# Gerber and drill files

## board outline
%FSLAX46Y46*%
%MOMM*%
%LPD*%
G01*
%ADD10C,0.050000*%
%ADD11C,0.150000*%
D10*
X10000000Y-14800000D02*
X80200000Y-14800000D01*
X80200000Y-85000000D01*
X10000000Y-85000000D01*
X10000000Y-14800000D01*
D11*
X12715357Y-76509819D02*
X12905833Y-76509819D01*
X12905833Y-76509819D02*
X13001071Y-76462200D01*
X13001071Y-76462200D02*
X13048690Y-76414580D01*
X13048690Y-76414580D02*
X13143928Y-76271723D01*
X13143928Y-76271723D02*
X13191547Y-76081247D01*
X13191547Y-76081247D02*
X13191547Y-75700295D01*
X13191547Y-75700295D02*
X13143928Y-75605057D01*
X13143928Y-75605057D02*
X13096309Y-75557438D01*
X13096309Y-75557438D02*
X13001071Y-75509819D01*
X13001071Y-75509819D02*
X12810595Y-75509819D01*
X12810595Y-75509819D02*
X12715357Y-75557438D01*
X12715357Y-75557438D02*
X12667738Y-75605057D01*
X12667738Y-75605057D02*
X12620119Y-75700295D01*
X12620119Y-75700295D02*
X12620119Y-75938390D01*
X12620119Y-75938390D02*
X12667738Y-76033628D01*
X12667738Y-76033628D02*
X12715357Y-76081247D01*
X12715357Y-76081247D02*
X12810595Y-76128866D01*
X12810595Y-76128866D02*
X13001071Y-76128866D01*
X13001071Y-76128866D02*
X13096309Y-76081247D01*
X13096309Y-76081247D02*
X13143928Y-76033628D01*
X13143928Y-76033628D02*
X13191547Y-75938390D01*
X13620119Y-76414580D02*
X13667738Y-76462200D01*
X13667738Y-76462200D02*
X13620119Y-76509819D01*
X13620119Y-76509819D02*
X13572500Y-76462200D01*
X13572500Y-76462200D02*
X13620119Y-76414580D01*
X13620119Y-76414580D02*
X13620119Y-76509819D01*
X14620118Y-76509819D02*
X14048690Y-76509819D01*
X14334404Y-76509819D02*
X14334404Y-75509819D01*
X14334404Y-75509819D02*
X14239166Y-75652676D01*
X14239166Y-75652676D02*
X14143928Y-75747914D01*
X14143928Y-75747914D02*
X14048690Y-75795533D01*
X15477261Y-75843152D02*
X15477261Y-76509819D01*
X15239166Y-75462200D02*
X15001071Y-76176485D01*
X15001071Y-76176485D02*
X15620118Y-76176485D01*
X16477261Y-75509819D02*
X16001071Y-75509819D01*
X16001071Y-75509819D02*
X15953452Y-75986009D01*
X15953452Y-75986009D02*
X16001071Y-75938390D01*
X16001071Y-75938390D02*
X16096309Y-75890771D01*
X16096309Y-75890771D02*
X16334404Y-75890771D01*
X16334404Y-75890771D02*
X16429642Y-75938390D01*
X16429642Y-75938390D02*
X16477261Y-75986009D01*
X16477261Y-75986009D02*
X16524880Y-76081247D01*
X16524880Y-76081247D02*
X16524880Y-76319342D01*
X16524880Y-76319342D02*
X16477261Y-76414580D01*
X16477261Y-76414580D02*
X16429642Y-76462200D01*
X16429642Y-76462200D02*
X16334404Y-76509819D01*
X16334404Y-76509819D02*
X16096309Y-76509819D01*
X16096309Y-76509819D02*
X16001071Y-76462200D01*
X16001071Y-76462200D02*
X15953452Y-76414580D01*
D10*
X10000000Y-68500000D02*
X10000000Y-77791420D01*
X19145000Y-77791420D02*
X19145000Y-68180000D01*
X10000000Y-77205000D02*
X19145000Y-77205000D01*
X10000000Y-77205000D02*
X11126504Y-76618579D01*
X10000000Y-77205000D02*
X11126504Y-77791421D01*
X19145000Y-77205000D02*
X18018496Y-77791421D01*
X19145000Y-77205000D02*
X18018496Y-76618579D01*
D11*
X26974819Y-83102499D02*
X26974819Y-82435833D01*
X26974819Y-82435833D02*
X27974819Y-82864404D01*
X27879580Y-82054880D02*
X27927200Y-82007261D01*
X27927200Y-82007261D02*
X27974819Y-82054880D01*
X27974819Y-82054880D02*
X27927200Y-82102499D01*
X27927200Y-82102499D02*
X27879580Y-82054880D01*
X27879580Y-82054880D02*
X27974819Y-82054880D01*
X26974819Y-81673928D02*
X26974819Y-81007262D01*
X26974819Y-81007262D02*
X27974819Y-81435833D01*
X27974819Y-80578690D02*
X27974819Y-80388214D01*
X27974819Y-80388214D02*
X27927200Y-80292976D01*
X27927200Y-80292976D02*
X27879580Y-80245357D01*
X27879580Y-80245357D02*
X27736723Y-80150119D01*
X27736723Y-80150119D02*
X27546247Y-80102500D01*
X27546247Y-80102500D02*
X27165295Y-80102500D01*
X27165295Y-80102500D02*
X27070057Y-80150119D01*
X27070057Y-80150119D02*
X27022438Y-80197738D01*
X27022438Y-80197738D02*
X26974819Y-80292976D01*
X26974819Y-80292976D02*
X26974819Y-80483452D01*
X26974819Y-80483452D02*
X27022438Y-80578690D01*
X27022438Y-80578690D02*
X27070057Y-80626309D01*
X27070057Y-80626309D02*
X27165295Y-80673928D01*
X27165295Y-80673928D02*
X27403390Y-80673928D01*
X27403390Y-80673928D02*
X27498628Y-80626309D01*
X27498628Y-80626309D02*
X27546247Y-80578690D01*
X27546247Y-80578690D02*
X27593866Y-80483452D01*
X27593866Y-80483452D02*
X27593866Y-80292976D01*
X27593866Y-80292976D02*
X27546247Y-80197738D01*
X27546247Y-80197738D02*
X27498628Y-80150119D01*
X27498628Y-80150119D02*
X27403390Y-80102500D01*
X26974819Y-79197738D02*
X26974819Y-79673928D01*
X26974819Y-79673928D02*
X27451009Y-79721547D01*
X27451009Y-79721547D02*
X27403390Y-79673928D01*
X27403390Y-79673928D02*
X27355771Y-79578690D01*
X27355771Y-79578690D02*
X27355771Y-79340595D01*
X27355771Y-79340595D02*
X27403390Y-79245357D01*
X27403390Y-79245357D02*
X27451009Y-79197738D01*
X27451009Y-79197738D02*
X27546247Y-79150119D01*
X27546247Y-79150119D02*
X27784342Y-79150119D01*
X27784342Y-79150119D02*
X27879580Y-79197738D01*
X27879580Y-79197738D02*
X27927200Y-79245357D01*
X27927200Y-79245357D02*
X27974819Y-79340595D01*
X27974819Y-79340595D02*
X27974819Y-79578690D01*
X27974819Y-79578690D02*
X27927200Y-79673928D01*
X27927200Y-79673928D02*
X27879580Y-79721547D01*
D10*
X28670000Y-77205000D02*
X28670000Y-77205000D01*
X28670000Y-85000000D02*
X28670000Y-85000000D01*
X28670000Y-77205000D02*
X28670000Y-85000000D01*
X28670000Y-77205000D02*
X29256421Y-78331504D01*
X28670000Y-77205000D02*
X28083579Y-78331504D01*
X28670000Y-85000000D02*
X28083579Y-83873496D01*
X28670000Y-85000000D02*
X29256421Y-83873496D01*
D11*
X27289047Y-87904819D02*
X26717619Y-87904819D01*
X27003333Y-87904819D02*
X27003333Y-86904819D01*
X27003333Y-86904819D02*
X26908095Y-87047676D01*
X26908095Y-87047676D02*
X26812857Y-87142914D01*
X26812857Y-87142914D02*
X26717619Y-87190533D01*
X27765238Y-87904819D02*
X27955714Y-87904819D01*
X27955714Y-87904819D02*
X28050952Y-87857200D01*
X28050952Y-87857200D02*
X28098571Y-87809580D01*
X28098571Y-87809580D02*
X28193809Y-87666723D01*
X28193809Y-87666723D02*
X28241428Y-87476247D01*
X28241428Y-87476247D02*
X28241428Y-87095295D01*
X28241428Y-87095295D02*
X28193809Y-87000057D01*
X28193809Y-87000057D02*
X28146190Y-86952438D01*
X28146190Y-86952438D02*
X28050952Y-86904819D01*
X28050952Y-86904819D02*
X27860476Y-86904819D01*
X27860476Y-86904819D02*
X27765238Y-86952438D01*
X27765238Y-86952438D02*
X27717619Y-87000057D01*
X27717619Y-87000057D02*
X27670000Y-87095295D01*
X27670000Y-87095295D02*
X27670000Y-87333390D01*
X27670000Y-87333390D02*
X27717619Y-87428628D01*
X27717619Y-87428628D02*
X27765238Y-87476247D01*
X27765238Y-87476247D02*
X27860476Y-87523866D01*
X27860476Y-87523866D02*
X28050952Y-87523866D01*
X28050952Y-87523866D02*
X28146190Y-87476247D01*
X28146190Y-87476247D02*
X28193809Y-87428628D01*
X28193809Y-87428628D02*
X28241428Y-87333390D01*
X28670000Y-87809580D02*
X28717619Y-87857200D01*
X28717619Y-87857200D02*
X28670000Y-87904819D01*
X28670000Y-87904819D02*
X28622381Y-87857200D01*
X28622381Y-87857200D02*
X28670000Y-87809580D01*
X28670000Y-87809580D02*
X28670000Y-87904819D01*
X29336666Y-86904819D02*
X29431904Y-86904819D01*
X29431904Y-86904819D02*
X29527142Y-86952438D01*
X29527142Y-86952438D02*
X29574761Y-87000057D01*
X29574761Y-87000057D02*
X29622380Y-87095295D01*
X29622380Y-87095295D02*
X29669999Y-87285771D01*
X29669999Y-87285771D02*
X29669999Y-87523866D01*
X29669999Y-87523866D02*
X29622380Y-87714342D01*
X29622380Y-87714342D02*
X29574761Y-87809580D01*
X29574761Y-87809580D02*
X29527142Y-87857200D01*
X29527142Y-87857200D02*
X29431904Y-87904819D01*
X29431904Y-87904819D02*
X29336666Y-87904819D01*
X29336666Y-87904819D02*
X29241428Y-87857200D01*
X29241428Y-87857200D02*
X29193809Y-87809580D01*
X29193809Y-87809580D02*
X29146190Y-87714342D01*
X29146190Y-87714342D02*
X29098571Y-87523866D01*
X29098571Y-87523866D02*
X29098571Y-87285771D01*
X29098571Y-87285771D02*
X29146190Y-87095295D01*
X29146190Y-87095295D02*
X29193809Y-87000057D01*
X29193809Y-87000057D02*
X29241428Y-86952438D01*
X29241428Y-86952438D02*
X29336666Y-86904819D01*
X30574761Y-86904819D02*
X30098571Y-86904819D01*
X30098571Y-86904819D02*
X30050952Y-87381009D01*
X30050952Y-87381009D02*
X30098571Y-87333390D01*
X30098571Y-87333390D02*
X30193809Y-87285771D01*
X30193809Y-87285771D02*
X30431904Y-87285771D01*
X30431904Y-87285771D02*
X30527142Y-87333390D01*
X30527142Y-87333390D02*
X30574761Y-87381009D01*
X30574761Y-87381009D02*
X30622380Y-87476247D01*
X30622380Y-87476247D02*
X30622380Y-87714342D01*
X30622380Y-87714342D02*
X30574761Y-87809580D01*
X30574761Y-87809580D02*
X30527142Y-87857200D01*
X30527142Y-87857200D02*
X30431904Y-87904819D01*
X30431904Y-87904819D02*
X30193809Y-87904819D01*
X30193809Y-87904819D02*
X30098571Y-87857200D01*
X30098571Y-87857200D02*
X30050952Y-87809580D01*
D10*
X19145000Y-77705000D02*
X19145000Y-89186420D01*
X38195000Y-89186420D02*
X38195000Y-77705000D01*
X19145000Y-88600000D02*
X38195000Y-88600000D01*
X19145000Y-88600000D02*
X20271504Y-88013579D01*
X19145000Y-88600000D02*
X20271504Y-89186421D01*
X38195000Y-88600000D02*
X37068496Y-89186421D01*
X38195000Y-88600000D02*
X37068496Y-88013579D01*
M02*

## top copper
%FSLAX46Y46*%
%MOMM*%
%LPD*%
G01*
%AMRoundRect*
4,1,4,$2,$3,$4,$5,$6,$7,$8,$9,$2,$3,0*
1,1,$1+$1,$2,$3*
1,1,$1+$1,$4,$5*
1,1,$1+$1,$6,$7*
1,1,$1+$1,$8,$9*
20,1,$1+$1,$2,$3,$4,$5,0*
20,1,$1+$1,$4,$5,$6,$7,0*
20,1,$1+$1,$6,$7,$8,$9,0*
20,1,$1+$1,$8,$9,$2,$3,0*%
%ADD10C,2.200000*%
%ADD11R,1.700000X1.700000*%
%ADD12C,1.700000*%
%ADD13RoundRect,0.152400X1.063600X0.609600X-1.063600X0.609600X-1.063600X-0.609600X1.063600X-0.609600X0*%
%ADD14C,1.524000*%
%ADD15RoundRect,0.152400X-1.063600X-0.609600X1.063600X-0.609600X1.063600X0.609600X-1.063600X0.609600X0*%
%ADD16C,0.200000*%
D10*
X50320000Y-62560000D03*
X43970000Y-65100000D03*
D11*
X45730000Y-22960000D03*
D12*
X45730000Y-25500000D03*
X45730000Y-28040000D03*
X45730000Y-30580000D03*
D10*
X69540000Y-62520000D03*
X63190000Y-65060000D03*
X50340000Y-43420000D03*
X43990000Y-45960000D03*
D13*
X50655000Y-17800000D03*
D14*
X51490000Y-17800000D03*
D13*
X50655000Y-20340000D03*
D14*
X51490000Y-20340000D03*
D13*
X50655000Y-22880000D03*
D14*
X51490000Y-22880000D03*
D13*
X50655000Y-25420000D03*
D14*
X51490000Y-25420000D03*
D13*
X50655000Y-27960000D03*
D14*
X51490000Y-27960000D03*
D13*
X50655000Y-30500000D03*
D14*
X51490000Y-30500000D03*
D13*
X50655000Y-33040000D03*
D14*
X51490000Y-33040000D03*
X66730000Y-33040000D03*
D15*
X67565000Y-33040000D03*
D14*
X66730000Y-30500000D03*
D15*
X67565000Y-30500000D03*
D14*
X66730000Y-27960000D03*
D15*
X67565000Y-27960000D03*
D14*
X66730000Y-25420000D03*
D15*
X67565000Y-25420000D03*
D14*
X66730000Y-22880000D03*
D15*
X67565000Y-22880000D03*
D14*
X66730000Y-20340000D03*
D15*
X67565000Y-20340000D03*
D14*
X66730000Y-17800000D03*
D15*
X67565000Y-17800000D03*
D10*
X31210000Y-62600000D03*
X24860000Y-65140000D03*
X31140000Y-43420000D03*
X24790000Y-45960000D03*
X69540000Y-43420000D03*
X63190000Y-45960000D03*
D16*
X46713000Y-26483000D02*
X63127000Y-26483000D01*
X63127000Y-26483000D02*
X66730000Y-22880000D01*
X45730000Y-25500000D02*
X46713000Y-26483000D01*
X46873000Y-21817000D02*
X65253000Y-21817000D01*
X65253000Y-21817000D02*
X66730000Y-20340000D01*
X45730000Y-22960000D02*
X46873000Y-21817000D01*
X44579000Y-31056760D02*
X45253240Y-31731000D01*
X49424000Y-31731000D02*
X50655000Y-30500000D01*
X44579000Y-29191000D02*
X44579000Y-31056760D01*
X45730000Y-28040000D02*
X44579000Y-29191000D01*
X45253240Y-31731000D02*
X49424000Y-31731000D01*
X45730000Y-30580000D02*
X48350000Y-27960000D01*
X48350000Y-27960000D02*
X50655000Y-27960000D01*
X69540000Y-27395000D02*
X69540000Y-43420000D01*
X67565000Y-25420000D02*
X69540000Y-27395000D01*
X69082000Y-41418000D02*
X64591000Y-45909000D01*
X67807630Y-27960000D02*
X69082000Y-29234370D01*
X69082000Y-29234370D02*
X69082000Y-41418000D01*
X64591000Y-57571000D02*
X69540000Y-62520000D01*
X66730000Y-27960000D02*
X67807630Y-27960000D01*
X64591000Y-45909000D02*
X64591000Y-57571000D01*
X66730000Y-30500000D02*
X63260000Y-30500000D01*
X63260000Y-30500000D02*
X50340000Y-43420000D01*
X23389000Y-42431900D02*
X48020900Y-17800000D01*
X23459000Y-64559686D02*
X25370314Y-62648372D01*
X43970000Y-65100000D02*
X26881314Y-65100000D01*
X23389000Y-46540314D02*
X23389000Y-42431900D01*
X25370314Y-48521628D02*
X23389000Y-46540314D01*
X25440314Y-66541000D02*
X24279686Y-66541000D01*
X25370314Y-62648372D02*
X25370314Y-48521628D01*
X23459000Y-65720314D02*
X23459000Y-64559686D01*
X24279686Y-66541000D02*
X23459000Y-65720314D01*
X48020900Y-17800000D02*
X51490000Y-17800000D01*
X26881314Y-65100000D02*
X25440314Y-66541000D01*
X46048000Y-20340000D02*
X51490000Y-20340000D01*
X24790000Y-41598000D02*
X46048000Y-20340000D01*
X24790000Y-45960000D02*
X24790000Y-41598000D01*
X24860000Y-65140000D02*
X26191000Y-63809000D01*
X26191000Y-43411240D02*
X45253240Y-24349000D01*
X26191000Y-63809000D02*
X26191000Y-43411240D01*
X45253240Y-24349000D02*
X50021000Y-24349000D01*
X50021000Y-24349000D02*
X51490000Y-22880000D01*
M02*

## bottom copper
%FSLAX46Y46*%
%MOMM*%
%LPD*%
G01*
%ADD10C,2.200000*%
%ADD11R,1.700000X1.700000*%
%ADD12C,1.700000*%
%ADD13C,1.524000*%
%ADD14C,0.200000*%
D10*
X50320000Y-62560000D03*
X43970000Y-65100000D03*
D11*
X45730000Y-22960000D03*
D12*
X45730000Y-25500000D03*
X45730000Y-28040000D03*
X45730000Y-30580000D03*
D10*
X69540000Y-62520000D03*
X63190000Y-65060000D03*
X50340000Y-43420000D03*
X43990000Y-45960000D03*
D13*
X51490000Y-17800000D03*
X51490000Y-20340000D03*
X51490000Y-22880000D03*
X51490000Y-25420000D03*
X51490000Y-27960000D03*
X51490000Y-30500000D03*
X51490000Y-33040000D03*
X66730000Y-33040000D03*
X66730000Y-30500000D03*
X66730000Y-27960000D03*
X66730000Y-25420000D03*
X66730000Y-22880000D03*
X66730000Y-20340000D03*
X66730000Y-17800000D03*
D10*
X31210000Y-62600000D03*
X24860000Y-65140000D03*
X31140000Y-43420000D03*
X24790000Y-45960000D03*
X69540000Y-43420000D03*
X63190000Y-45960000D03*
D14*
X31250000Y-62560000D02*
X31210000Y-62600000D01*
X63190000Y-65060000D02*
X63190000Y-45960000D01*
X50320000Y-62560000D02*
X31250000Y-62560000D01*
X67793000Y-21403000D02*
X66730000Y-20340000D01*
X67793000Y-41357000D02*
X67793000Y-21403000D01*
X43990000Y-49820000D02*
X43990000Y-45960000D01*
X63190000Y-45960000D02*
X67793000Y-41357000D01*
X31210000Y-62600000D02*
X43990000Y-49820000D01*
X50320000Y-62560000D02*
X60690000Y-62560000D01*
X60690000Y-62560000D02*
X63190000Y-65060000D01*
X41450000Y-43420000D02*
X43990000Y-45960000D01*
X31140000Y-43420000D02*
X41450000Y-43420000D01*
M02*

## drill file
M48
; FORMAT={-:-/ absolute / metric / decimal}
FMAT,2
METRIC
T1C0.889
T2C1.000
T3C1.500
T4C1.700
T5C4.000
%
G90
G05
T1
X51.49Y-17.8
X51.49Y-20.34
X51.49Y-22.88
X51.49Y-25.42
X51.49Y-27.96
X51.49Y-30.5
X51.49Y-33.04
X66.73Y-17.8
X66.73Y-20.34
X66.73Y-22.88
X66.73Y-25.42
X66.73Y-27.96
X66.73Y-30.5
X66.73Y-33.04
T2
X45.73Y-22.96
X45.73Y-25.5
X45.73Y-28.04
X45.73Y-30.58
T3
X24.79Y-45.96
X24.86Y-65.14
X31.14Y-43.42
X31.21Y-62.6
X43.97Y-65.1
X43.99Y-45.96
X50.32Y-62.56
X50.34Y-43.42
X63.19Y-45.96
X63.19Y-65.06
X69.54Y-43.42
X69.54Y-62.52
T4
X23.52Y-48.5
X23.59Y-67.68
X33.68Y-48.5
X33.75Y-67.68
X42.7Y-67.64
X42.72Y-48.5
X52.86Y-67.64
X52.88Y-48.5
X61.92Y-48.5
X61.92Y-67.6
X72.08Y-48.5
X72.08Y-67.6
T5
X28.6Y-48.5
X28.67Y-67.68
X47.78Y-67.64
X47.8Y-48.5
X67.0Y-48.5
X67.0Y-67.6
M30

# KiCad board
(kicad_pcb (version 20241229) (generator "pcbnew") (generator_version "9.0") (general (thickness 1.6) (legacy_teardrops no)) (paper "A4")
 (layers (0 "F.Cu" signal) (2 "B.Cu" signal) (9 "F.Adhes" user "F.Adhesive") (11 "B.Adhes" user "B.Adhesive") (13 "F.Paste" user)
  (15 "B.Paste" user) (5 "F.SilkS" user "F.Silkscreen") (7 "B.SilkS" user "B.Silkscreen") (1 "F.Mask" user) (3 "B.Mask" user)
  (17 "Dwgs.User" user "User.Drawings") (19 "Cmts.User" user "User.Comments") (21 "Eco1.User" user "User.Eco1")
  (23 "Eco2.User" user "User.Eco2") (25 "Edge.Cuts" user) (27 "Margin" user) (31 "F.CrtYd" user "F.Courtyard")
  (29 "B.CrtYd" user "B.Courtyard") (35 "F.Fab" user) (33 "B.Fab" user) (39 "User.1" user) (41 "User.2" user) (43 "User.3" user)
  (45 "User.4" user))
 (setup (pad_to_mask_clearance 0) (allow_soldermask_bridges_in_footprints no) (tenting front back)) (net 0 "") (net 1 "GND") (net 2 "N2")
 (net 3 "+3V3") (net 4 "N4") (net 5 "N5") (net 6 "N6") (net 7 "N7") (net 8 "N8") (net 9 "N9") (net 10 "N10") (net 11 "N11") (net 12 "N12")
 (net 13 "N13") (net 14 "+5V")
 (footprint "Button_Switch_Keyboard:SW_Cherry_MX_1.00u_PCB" (layer "F.Cu") (at 50.32 62.56)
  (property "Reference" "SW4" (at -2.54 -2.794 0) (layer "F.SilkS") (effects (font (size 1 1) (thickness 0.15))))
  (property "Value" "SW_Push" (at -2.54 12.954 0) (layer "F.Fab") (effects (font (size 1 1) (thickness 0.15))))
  (pad "" np_thru_hole circle (at -7.62 5.08) (size 1.7 1.7) (drill 1.7) (layers "*.Cu" "*.Mask"))
  (pad "" np_thru_hole circle (at -2.54 5.08) (size 4 4) (drill 4) (layers "*.Cu" "*.Mask"))
  (pad "" np_thru_hole circle (at 2.54 5.08) (size 1.7 1.7) (drill 1.7) (layers "*.Cu" "*.Mask"))
  (pad "1" thru_hole circle (at 0 0) (size 2.2 2.2) (drill 1.5) (layers "*.Cu" "*.Mask") (remove_unused_layers no) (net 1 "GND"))
  (pad "2" thru_hole circle (at -6.35 2.54) (size 2.2 2.2) (drill 1.5) (layers "*.Cu" "*.Mask") (remove_unused_layers no) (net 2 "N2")))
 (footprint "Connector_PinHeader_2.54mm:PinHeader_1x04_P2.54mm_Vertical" (layer "F.Cu") (at 45.73 22.96)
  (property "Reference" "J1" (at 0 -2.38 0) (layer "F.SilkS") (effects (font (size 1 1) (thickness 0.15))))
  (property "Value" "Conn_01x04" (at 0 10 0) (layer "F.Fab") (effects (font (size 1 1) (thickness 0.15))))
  (pad "1" thru_hole rect (at 0 0) (size 1.7 1.7) (drill 1) (layers "*.Cu" "*.Mask") (remove_unused_layers no) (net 1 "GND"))
  (pad "2" thru_hole circle (at 0 2.54) (size 1.7 1.7) (drill 1) (layers "*.Cu" "*.Mask") (remove_unused_layers no) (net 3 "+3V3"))
  (pad "3" thru_hole circle (at 0 5.08) (size 1.7 1.7) (drill 1) (layers "*.Cu" "*.Mask") (remove_unused_layers no) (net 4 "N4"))
  (pad "4" thru_hole circle (at 0 7.62) (size 1.7 1.7) (drill 1) (layers "*.Cu" "*.Mask") (remove_unused_layers no) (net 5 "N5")))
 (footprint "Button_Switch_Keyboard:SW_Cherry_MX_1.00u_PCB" (layer "F.Cu") (at 69.54 62.52)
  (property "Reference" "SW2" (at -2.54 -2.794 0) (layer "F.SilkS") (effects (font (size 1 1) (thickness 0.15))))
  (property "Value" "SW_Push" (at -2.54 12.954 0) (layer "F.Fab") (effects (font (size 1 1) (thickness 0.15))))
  (pad "" np_thru_hole circle (at -7.62 5.08) (size 1.7 1.7) (drill 1.7) (layers "*.Cu" "*.Mask"))
  (pad "" np_thru_hole circle (at -2.54 5.08) (size 4 4) (drill 4) (layers "*.Cu" "*.Mask"))
  (pad "" np_thru_hole circle (at 2.54 5.08) (size 1.7 1.7) (drill 1.7) (layers "*.Cu" "*.Mask"))
  (pad "1" thru_hole circle (at 0 0) (size 2.2 2.2) (drill 1.5) (layers "*.Cu" "*.Mask") (remove_unused_layers no) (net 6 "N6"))
  (pad "2" thru_hole circle (at -6.35 2.54) (size 2.2 2.2) (drill 1.5) (layers "*.Cu" "*.Mask") (remove_unused_layers no) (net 1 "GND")))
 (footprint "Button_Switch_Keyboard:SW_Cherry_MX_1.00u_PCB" (layer "F.Cu") (at 50.34 43.42)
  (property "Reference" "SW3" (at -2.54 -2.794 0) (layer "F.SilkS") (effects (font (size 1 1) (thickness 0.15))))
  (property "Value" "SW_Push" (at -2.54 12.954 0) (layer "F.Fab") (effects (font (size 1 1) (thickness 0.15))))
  (pad "" np_thru_hole circle (at -7.62 5.08) (size 1.7 1.7) (drill 1.7) (layers "*.Cu" "*.Mask"))
  (pad "" np_thru_hole circle (at -2.54 5.08) (size 4 4) (drill 4) (layers "*.Cu" "*.Mask"))
  (pad "" np_thru_hole circle (at 2.54 5.08) (size 1.7 1.7) (drill 1.7) (layers "*.Cu" "*.Mask"))
  (pad "1" thru_hole circle (at 0 0) (size 2.2 2.2) (drill 1.5) (layers "*.Cu" "*.Mask") (remove_unused_layers no) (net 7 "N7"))
  (pad "2" thru_hole circle (at -6.35 2.54) (size 2.2 2.2) (drill 1.5) (layers "*.Cu" "*.Mask") (remove_unused_layers no) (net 1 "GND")))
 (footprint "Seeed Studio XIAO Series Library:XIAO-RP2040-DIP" (layer "F.Cu") (at 59.11 25.42)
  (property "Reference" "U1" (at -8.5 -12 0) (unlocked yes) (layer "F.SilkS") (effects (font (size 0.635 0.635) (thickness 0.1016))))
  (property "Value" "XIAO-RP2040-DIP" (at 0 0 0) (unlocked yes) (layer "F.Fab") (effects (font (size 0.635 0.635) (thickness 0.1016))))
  (pad "1" smd roundrect (at -8.455 -7.62 180) (size 2.432 1.524) (layers "F.Cu" "F.Mask") (roundrect_rratio 0.1) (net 2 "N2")
   (thermal_bridge_angle 45))
  (pad "1" thru_hole circle (at -7.62 -7.62 180) (size 1.524 1.524) (drill 0.889) (layers "*.Cu" "*.Mask") (remove_unused_layers no)
   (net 2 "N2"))
  (pad "2" smd roundrect (at -8.455 -5.08 180) (size 2.432 1.524) (layers "F.Cu" "F.Mask") (roundrect_rratio 0.1) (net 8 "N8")
   (thermal_bridge_angle 45))
  (pad "2" thru_hole circle (at -7.62 -5.08 180) (size 1.524 1.524) (drill 0.889) (layers "*.Cu" "*.Mask") (remove_unused_layers no)
   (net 8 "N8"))
  (pad "3" smd roundrect (at -8.455 -2.54 180) (size 2.432 1.524) (layers "F.Cu" "F.Mask") (roundrect_rratio 0.1) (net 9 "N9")
   (thermal_bridge_angle 45))
  (pad "3" thru_hole circle (at -7.62 -2.54 180) (size 1.524 1.524) (drill 0.889) (layers "*.Cu" "*.Mask") (remove_unused_layers no)
   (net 9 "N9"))
  (pad "4" smd roundrect (at -8.455 0 180) (size 2.432 1.524) (layers "F.Cu" "F.Mask") (roundrect_rratio 0.1) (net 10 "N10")
   (thermal_bridge_angle 45))
  (pad "4" thru_hole circle (at -7.62 0 180) (size 1.524 1.524) (drill 0.889) (layers "*.Cu" "*.Mask") (remove_unused_layers no)
   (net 10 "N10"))
  (pad "5" smd roundrect (at -8.455 2.54 180) (size 2.432 1.524) (layers "F.Cu" "F.Mask") (roundrect_rratio 0.1) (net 5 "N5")
   (thermal_bridge_angle 45))
  (pad "5" thru_hole circle (at -7.62 2.54 180) (size 1.524 1.524) (drill 0.889) (layers "*.Cu" "*.Mask") (remove_unused_layers no)
   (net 5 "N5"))
  (pad "6" smd roundrect (at -8.455 5.08 180) (size 2.432 1.524) (layers "F.Cu" "F.Mask") (roundrect_rratio 0.1) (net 4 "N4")
   (thermal_bridge_angle 45))
  (pad "6" thru_hole circle (at -7.62 5.08 180) (size 1.524 1.524) (drill 0.889) (layers "*.Cu" "*.Mask") (remove_unused_layers no)
   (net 4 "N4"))
  (pad "7" smd roundrect (at -8.455 7.62 180) (size 2.432 1.524) (layers "F.Cu" "F.Mask") (roundrect_rratio 0.1) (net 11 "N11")
   (thermal_bridge_angle 45))
  (pad "7" thru_hole circle (at -7.62 7.62 180) (size 1.524 1.524) (drill 0.889) (layers "*.Cu" "*.Mask") (remove_unused_layers no)
   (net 11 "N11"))
  (pad "8" thru_hole circle (at 7.62 7.62) (size 1.524 1.524) (drill 0.889) (layers "*.Cu" "*.Mask") (remove_unused_layers no)
   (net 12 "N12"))
  (pad "8" smd roundrect (at 8.455 7.62) (size 2.432 1.524) (layers "F.Cu" "F.Mask") (roundrect_rratio 0.1) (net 12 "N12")
   (thermal_bridge_angle 45))
  (pad "9" thru_hole circle (at 7.62 5.08) (size 1.524 1.524) (drill 0.889) (layers "*.Cu" "*.Mask") (remove_unused_layers no) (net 7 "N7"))
  (pad "9" smd roundrect (at 8.455 5.08) (size 2.432 1.524) (layers "F.Cu" "F.Mask") (roundrect_rratio 0.1) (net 7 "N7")
   (thermal_bridge_angle 45))
  (pad "10" thru_hole circle (at 7.62 2.54) (size 1.524 1.524) (drill 0.889) (layers "*.Cu" "*.Mask") (remove_unused_layers no) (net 6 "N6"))
  (pad "10" smd roundrect (at 8.455 2.54) (size 2.432 1.524) (layers "F.Cu" "F.Mask") (roundrect_rratio 0.1) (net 6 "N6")
   (thermal_bridge_angle 45))
  (pad "11" thru_hole circle (at 7.62 0) (size 1.524 1.524) (drill 0.889) (layers "*.Cu" "*.Mask") (remove_unused_layers no) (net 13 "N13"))
  (pad "11" smd roundrect (at 8.455 0) (size 2.432 1.524) (layers "F.Cu" "F.Mask") (roundrect_rratio 0.1) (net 13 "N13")
   (thermal_bridge_angle 45))
  (pad "12" thru_hole circle (at 7.62 -2.54) (size 1.524 1.524) (drill 0.889) (layers "*.Cu" "*.Mask") (remove_unused_layers no)
   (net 3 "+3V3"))
  (pad "12" smd roundrect (at 8.455 -2.54) (size 2.432 1.524) (layers "F.Cu" "F.Mask") (roundrect_rratio 0.1) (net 3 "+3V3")
   (thermal_bridge_angle 45))
  (pad "13" thru_hole circle (at 7.62 -5.08) (size 1.524 1.524) (drill 0.889) (layers "*.Cu" "*.Mask") (remove_unused_layers no)
   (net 1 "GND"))
  (pad "13" smd roundrect (at 8.455 -5.08) (size 2.432 1.524) (layers "F.Cu" "F.Mask") (roundrect_rratio 0.1) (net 1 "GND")
   (thermal_bridge_angle 45))
  (pad "14" thru_hole circle (at 7.62 -7.62) (size 1.524 1.524) (drill 0.889) (layers "*.Cu" "*.Mask") (remove_unused_layers no)
   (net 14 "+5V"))
  (pad "14" smd roundrect (at 8.455 -7.62) (size 2.432 1.524) (layers "F.Cu" "F.Mask") (roundrect_rratio 0.1) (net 14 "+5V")
   (thermal_bridge_angle 45)))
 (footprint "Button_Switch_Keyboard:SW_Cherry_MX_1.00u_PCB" (layer "F.Cu") (at 31.21 62.6)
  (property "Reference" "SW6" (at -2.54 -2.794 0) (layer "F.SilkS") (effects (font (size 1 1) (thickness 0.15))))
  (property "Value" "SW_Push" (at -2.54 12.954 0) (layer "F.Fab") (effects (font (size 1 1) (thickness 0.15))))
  (pad "" np_thru_hole circle (at -7.62 5.08) (size 1.7 1.7) (drill 1.7) (layers "*.Cu" "*.Mask"))
  (pad "" np_thru_hole circle (at -2.54 5.08) (size 4 4) (drill 4) (layers "*.Cu" "*.Mask"))
  (pad "" np_thru_hole circle (at 2.54 5.08) (size 1.7 1.7) (drill 1.7) (layers "*.Cu" "*.Mask"))
  (pad "1" thru_hole circle (at 0 0) (size 2.2 2.2) (drill 1.5) (layers "*.Cu" "*.Mask") (remove_unused_layers no) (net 1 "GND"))
  (pad "2" thru_hole circle (at -6.35 2.54) (size 2.2 2.2) (drill 1.5) (layers "*.Cu" "*.Mask") (remove_unused_layers no) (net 9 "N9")))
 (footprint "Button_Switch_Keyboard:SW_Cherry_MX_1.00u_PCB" (layer "F.Cu") (at 31.14 43.42)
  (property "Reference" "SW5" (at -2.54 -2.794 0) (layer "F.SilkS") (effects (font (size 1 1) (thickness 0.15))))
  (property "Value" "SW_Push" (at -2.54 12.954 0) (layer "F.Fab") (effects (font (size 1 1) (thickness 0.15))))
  (pad "" np_thru_hole circle (at -7.62 5.08) (size 1.7 1.7) (drill 1.7) (layers "*.Cu" "*.Mask"))
  (pad "" np_thru_hole circle (at -2.54 5.08) (size 4 4) (drill 4) (layers "*.Cu" "*.Mask"))
  (pad "" np_thru_hole circle (at 2.54 5.08) (size 1.7 1.7) (drill 1.7) (layers "*.Cu" "*.Mask"))
  (pad "1" thru_hole circle (at 0 0) (size 2.2 2.2) (drill 1.5) (layers "*.Cu" "*.Mask") (remove_unused_layers no) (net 1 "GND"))
  (pad "2" thru_hole circle (at -6.35 2.54) (size 2.2 2.2) (drill 1.5) (layers "*.Cu" "*.Mask") (remove_unused_layers no) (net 8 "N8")))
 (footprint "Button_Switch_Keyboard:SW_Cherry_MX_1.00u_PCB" (layer "F.Cu") (at 69.54 43.42)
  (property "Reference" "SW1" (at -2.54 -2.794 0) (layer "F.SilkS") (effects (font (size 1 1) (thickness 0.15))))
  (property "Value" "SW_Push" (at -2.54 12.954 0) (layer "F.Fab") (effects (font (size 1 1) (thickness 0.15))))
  (pad "" np_thru_hole circle (at -7.62 5.08) (size 1.7 1.7) (drill 1.7) (layers "*.Cu" "*.Mask"))
  (pad "" np_thru_hole circle (at -2.54 5.08) (size 4 4) (drill 4) (layers "*.Cu" "*.Mask"))
  (pad "" np_thru_hole circle (at 2.54 5.08) (size 1.7 1.7) (drill 1.7) (layers "*.Cu" "*.Mask"))
  (pad "1" thru_hole circle (at 0 0) (size 2.2 2.2) (drill 1.5) (layers "*.Cu" "*.Mask") (remove_unused_layers no) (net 13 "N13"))
  (pad "2" thru_hole circle (at -6.35 2.54) (size 2.2 2.2) (drill 1.5) (layers "*.Cu" "*.Mask") (remove_unused_layers no) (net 1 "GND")))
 (gr_rect (start 10 14.8) (end 80.2 85) (stroke (width 0.05) (type default)) (fill no) (layer "Edge.Cuts"))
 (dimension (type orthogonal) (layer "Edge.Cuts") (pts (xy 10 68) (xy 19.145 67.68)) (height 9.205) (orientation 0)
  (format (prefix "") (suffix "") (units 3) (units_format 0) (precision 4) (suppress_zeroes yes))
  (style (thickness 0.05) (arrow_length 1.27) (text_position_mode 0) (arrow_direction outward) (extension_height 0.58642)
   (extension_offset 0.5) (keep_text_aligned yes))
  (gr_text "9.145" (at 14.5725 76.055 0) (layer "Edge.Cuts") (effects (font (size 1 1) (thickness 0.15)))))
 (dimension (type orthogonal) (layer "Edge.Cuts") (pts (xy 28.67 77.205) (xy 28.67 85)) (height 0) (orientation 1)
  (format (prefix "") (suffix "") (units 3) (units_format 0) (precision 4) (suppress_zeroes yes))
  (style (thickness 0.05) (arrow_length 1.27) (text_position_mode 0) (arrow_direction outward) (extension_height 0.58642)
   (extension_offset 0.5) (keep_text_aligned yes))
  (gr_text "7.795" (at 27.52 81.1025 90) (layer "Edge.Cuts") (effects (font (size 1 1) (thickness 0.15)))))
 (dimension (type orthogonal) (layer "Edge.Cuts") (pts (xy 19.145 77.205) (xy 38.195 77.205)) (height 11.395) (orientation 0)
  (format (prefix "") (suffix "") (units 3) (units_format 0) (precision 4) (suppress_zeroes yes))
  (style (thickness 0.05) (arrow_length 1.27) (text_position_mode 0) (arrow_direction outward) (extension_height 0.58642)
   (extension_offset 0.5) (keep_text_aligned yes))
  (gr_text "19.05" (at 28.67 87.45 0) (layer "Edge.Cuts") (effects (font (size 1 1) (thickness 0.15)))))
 (segment (start 46.713 26.483) (end 63.127 26.483) (width 0.2) (layer "F.Cu") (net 3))
 (segment (start 63.127 26.483) (end 66.73 22.88) (width 0.2) (layer "F.Cu") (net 3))
 (segment (start 45.73 25.5) (end 46.713 26.483) (width 0.2) (layer "F.Cu") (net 3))
 (segment (start 46.873 21.817) (end 65.253 21.817) (width 0.2) (layer "F.Cu") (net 1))
 (segment (start 65.253 21.817) (end 66.73 20.34) (width 0.2) (layer "F.Cu") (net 1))
 (segment (start 45.73 22.96) (end 46.873 21.817) (width 0.2) (layer "F.Cu") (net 1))
 (segment (start 31.25 62.56) (end 31.21 62.6) (width 0.2) (layer "B.Cu") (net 1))
 (segment (start 63.19 65.06) (end 63.19 45.96) (width 0.2) (layer "B.Cu") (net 1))
 (segment (start 50.32 62.56) (end 31.25 62.56) (width 0.2) (layer "B.Cu") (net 1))
 (segment (start 67.793 21.403) (end 66.73 20.34) (width 0.2) (layer "B.Cu") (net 1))
 (segment (start 67.793 41.357) (end 67.793 21.403) (width 0.2) (layer "B.Cu") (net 1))
 (segment (start 43.99 49.82) (end 43.99 45.96) (width 0.2) (layer "B.Cu") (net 1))
 (segment (start 63.19 45.96) (end 67.793 41.357) (width 0.2) (layer "B.Cu") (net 1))
 (segment (start 31.21 62.6) (end 43.99 49.82) (width 0.2) (layer "B.Cu") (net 1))
 (segment (start 50.32 62.56) (end 60.69 62.56) (width 0.2) (layer "B.Cu") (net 1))
 (segment (start 60.69 62.56) (end 63.19 65.06) (width 0.2) (layer "B.Cu") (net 1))
 (segment (start 41.45 43.42) (end 43.99 45.96) (width 0.2) (layer "B.Cu") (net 1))
 (segment (start 31.14 43.42) (end 41.45 43.42) (width 0.2) (layer "B.Cu") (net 1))
 (segment (start 44.579 31.05676) (end 45.25324 31.731) (width 0.2) (layer "F.Cu") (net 4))
 (segment (start 49.424 31.731) (end 50.655 30.5) (width 0.2) (layer "F.Cu") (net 4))
 (segment (start 44.579 29.191) (end 44.579 31.05676) (width 0.2) (layer "F.Cu") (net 4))
 (segment (start 45.73 28.04) (end 44.579 29.191) (width 0.2) (layer "F.Cu") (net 4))
 (segment (start 45.25324 31.731) (end 49.424 31.731) (width 0.2) (layer "F.Cu") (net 4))
 (segment (start 45.73 30.58) (end 48.35 27.96) (width 0.2) (layer "F.Cu") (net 5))
 (segment (start 48.35 27.96) (end 50.655 27.96) (width 0.2) (layer "F.Cu") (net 5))
 (segment (start 69.54 27.395) (end 69.54 43.42) (width 0.2) (layer "F.Cu") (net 13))
 (segment (start 67.565 25.42) (end 69.54 27.395) (width 0.2) (layer "F.Cu") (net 13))
 (segment (start 69.082 41.418) (end 64.591 45.909) (width 0.2) (layer "F.Cu") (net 6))
 (segment (start 67.80763 27.96) (end 69.082 29.23437) (width 0.2) (layer "F.Cu") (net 6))
 (segment (start 69.082 29.23437) (end 69.082 41.418) (width 0.2) (layer "F.Cu") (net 6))
 (segment (start 64.591 57.571) (end 69.54 62.52) (width 0.2) (layer "F.Cu") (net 6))
 (segment (start 66.73 27.96) (end 67.80763 27.96) (width 0.2) (layer "F.Cu") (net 6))
 (segment (start 64.591 45.909) (end 64.591 57.571) (width 0.2) (layer "F.Cu") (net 6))
 (segment (start 66.73 30.5) (end 63.26 30.5) (width 0.2) (layer "F.Cu") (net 7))
 (segment (start 63.26 30.5) (end 50.34 43.42) (width 0.2) (layer "F.Cu") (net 7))
 (segment (start 23.389 42.4319) (end 48.0209 17.8) (width 0.2) (layer "F.Cu") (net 2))
 (segment (start 23.459 64.559686) (end 25.370314 62.648372) (width 0.2) (layer "F.Cu") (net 2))
 (segment (start 43.97 65.1) (end 26.881314 65.1) (width 0.2) (layer "F.Cu") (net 2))
 (segment (start 23.389 46.540314) (end 23.389 42.4319) (width 0.2) (layer "F.Cu") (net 2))
 (segment (start 25.370314 48.521628) (end 23.389 46.540314) (width 0.2) (layer "F.Cu") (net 2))
 (segment (start 25.440314 66.541) (end 24.279686 66.541) (width 0.2) (layer "F.Cu") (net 2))
 (segment (start 25.370314 62.648372) (end 25.370314 48.521628) (width 0.2) (layer "F.Cu") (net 2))
 (segment (start 23.459 65.720314) (end 23.459 64.559686) (width 0.2) (layer "F.Cu") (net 2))
 (segment (start 24.279686 66.541) (end 23.459 65.720314) (width 0.2) (layer "F.Cu") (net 2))
 (segment (start 48.0209 17.8) (end 51.49 17.8) (width 0.2) (layer "F.Cu") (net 2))
 (segment (start 26.881314 65.1) (end 25.440314 66.541) (width 0.2) (layer "F.Cu") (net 2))
 (segment (start 46.048 20.34) (end 51.49 20.34) (width 0.2) (layer "F.Cu") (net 8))
 (segment (start 24.79 41.598) (end 46.048 20.34) (width 0.2) (layer "F.Cu") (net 8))
 (segment (start 24.79 45.96) (end 24.79 41.598) (width 0.2) (layer "F.Cu") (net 8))
 (segment (start 24.86 65.14) (end 26.191 63.809) (width 0.2) (layer "F.Cu") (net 9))
 (segment (start 26.191 43.41124) (end 45.25324 24.349) (width 0.2) (layer "F.Cu") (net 9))
 (segment (start 26.191 63.809) (end 26.191 43.41124) (width 0.2) (layer "F.Cu") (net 9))
 (segment (start 45.25324 24.349) (end 50.021 24.349) (width 0.2) (layer "F.Cu") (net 9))
 (segment (start 50.021 24.349) (end 51.49 22.88) (width 0.2) (layer "F.Cu") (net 9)))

